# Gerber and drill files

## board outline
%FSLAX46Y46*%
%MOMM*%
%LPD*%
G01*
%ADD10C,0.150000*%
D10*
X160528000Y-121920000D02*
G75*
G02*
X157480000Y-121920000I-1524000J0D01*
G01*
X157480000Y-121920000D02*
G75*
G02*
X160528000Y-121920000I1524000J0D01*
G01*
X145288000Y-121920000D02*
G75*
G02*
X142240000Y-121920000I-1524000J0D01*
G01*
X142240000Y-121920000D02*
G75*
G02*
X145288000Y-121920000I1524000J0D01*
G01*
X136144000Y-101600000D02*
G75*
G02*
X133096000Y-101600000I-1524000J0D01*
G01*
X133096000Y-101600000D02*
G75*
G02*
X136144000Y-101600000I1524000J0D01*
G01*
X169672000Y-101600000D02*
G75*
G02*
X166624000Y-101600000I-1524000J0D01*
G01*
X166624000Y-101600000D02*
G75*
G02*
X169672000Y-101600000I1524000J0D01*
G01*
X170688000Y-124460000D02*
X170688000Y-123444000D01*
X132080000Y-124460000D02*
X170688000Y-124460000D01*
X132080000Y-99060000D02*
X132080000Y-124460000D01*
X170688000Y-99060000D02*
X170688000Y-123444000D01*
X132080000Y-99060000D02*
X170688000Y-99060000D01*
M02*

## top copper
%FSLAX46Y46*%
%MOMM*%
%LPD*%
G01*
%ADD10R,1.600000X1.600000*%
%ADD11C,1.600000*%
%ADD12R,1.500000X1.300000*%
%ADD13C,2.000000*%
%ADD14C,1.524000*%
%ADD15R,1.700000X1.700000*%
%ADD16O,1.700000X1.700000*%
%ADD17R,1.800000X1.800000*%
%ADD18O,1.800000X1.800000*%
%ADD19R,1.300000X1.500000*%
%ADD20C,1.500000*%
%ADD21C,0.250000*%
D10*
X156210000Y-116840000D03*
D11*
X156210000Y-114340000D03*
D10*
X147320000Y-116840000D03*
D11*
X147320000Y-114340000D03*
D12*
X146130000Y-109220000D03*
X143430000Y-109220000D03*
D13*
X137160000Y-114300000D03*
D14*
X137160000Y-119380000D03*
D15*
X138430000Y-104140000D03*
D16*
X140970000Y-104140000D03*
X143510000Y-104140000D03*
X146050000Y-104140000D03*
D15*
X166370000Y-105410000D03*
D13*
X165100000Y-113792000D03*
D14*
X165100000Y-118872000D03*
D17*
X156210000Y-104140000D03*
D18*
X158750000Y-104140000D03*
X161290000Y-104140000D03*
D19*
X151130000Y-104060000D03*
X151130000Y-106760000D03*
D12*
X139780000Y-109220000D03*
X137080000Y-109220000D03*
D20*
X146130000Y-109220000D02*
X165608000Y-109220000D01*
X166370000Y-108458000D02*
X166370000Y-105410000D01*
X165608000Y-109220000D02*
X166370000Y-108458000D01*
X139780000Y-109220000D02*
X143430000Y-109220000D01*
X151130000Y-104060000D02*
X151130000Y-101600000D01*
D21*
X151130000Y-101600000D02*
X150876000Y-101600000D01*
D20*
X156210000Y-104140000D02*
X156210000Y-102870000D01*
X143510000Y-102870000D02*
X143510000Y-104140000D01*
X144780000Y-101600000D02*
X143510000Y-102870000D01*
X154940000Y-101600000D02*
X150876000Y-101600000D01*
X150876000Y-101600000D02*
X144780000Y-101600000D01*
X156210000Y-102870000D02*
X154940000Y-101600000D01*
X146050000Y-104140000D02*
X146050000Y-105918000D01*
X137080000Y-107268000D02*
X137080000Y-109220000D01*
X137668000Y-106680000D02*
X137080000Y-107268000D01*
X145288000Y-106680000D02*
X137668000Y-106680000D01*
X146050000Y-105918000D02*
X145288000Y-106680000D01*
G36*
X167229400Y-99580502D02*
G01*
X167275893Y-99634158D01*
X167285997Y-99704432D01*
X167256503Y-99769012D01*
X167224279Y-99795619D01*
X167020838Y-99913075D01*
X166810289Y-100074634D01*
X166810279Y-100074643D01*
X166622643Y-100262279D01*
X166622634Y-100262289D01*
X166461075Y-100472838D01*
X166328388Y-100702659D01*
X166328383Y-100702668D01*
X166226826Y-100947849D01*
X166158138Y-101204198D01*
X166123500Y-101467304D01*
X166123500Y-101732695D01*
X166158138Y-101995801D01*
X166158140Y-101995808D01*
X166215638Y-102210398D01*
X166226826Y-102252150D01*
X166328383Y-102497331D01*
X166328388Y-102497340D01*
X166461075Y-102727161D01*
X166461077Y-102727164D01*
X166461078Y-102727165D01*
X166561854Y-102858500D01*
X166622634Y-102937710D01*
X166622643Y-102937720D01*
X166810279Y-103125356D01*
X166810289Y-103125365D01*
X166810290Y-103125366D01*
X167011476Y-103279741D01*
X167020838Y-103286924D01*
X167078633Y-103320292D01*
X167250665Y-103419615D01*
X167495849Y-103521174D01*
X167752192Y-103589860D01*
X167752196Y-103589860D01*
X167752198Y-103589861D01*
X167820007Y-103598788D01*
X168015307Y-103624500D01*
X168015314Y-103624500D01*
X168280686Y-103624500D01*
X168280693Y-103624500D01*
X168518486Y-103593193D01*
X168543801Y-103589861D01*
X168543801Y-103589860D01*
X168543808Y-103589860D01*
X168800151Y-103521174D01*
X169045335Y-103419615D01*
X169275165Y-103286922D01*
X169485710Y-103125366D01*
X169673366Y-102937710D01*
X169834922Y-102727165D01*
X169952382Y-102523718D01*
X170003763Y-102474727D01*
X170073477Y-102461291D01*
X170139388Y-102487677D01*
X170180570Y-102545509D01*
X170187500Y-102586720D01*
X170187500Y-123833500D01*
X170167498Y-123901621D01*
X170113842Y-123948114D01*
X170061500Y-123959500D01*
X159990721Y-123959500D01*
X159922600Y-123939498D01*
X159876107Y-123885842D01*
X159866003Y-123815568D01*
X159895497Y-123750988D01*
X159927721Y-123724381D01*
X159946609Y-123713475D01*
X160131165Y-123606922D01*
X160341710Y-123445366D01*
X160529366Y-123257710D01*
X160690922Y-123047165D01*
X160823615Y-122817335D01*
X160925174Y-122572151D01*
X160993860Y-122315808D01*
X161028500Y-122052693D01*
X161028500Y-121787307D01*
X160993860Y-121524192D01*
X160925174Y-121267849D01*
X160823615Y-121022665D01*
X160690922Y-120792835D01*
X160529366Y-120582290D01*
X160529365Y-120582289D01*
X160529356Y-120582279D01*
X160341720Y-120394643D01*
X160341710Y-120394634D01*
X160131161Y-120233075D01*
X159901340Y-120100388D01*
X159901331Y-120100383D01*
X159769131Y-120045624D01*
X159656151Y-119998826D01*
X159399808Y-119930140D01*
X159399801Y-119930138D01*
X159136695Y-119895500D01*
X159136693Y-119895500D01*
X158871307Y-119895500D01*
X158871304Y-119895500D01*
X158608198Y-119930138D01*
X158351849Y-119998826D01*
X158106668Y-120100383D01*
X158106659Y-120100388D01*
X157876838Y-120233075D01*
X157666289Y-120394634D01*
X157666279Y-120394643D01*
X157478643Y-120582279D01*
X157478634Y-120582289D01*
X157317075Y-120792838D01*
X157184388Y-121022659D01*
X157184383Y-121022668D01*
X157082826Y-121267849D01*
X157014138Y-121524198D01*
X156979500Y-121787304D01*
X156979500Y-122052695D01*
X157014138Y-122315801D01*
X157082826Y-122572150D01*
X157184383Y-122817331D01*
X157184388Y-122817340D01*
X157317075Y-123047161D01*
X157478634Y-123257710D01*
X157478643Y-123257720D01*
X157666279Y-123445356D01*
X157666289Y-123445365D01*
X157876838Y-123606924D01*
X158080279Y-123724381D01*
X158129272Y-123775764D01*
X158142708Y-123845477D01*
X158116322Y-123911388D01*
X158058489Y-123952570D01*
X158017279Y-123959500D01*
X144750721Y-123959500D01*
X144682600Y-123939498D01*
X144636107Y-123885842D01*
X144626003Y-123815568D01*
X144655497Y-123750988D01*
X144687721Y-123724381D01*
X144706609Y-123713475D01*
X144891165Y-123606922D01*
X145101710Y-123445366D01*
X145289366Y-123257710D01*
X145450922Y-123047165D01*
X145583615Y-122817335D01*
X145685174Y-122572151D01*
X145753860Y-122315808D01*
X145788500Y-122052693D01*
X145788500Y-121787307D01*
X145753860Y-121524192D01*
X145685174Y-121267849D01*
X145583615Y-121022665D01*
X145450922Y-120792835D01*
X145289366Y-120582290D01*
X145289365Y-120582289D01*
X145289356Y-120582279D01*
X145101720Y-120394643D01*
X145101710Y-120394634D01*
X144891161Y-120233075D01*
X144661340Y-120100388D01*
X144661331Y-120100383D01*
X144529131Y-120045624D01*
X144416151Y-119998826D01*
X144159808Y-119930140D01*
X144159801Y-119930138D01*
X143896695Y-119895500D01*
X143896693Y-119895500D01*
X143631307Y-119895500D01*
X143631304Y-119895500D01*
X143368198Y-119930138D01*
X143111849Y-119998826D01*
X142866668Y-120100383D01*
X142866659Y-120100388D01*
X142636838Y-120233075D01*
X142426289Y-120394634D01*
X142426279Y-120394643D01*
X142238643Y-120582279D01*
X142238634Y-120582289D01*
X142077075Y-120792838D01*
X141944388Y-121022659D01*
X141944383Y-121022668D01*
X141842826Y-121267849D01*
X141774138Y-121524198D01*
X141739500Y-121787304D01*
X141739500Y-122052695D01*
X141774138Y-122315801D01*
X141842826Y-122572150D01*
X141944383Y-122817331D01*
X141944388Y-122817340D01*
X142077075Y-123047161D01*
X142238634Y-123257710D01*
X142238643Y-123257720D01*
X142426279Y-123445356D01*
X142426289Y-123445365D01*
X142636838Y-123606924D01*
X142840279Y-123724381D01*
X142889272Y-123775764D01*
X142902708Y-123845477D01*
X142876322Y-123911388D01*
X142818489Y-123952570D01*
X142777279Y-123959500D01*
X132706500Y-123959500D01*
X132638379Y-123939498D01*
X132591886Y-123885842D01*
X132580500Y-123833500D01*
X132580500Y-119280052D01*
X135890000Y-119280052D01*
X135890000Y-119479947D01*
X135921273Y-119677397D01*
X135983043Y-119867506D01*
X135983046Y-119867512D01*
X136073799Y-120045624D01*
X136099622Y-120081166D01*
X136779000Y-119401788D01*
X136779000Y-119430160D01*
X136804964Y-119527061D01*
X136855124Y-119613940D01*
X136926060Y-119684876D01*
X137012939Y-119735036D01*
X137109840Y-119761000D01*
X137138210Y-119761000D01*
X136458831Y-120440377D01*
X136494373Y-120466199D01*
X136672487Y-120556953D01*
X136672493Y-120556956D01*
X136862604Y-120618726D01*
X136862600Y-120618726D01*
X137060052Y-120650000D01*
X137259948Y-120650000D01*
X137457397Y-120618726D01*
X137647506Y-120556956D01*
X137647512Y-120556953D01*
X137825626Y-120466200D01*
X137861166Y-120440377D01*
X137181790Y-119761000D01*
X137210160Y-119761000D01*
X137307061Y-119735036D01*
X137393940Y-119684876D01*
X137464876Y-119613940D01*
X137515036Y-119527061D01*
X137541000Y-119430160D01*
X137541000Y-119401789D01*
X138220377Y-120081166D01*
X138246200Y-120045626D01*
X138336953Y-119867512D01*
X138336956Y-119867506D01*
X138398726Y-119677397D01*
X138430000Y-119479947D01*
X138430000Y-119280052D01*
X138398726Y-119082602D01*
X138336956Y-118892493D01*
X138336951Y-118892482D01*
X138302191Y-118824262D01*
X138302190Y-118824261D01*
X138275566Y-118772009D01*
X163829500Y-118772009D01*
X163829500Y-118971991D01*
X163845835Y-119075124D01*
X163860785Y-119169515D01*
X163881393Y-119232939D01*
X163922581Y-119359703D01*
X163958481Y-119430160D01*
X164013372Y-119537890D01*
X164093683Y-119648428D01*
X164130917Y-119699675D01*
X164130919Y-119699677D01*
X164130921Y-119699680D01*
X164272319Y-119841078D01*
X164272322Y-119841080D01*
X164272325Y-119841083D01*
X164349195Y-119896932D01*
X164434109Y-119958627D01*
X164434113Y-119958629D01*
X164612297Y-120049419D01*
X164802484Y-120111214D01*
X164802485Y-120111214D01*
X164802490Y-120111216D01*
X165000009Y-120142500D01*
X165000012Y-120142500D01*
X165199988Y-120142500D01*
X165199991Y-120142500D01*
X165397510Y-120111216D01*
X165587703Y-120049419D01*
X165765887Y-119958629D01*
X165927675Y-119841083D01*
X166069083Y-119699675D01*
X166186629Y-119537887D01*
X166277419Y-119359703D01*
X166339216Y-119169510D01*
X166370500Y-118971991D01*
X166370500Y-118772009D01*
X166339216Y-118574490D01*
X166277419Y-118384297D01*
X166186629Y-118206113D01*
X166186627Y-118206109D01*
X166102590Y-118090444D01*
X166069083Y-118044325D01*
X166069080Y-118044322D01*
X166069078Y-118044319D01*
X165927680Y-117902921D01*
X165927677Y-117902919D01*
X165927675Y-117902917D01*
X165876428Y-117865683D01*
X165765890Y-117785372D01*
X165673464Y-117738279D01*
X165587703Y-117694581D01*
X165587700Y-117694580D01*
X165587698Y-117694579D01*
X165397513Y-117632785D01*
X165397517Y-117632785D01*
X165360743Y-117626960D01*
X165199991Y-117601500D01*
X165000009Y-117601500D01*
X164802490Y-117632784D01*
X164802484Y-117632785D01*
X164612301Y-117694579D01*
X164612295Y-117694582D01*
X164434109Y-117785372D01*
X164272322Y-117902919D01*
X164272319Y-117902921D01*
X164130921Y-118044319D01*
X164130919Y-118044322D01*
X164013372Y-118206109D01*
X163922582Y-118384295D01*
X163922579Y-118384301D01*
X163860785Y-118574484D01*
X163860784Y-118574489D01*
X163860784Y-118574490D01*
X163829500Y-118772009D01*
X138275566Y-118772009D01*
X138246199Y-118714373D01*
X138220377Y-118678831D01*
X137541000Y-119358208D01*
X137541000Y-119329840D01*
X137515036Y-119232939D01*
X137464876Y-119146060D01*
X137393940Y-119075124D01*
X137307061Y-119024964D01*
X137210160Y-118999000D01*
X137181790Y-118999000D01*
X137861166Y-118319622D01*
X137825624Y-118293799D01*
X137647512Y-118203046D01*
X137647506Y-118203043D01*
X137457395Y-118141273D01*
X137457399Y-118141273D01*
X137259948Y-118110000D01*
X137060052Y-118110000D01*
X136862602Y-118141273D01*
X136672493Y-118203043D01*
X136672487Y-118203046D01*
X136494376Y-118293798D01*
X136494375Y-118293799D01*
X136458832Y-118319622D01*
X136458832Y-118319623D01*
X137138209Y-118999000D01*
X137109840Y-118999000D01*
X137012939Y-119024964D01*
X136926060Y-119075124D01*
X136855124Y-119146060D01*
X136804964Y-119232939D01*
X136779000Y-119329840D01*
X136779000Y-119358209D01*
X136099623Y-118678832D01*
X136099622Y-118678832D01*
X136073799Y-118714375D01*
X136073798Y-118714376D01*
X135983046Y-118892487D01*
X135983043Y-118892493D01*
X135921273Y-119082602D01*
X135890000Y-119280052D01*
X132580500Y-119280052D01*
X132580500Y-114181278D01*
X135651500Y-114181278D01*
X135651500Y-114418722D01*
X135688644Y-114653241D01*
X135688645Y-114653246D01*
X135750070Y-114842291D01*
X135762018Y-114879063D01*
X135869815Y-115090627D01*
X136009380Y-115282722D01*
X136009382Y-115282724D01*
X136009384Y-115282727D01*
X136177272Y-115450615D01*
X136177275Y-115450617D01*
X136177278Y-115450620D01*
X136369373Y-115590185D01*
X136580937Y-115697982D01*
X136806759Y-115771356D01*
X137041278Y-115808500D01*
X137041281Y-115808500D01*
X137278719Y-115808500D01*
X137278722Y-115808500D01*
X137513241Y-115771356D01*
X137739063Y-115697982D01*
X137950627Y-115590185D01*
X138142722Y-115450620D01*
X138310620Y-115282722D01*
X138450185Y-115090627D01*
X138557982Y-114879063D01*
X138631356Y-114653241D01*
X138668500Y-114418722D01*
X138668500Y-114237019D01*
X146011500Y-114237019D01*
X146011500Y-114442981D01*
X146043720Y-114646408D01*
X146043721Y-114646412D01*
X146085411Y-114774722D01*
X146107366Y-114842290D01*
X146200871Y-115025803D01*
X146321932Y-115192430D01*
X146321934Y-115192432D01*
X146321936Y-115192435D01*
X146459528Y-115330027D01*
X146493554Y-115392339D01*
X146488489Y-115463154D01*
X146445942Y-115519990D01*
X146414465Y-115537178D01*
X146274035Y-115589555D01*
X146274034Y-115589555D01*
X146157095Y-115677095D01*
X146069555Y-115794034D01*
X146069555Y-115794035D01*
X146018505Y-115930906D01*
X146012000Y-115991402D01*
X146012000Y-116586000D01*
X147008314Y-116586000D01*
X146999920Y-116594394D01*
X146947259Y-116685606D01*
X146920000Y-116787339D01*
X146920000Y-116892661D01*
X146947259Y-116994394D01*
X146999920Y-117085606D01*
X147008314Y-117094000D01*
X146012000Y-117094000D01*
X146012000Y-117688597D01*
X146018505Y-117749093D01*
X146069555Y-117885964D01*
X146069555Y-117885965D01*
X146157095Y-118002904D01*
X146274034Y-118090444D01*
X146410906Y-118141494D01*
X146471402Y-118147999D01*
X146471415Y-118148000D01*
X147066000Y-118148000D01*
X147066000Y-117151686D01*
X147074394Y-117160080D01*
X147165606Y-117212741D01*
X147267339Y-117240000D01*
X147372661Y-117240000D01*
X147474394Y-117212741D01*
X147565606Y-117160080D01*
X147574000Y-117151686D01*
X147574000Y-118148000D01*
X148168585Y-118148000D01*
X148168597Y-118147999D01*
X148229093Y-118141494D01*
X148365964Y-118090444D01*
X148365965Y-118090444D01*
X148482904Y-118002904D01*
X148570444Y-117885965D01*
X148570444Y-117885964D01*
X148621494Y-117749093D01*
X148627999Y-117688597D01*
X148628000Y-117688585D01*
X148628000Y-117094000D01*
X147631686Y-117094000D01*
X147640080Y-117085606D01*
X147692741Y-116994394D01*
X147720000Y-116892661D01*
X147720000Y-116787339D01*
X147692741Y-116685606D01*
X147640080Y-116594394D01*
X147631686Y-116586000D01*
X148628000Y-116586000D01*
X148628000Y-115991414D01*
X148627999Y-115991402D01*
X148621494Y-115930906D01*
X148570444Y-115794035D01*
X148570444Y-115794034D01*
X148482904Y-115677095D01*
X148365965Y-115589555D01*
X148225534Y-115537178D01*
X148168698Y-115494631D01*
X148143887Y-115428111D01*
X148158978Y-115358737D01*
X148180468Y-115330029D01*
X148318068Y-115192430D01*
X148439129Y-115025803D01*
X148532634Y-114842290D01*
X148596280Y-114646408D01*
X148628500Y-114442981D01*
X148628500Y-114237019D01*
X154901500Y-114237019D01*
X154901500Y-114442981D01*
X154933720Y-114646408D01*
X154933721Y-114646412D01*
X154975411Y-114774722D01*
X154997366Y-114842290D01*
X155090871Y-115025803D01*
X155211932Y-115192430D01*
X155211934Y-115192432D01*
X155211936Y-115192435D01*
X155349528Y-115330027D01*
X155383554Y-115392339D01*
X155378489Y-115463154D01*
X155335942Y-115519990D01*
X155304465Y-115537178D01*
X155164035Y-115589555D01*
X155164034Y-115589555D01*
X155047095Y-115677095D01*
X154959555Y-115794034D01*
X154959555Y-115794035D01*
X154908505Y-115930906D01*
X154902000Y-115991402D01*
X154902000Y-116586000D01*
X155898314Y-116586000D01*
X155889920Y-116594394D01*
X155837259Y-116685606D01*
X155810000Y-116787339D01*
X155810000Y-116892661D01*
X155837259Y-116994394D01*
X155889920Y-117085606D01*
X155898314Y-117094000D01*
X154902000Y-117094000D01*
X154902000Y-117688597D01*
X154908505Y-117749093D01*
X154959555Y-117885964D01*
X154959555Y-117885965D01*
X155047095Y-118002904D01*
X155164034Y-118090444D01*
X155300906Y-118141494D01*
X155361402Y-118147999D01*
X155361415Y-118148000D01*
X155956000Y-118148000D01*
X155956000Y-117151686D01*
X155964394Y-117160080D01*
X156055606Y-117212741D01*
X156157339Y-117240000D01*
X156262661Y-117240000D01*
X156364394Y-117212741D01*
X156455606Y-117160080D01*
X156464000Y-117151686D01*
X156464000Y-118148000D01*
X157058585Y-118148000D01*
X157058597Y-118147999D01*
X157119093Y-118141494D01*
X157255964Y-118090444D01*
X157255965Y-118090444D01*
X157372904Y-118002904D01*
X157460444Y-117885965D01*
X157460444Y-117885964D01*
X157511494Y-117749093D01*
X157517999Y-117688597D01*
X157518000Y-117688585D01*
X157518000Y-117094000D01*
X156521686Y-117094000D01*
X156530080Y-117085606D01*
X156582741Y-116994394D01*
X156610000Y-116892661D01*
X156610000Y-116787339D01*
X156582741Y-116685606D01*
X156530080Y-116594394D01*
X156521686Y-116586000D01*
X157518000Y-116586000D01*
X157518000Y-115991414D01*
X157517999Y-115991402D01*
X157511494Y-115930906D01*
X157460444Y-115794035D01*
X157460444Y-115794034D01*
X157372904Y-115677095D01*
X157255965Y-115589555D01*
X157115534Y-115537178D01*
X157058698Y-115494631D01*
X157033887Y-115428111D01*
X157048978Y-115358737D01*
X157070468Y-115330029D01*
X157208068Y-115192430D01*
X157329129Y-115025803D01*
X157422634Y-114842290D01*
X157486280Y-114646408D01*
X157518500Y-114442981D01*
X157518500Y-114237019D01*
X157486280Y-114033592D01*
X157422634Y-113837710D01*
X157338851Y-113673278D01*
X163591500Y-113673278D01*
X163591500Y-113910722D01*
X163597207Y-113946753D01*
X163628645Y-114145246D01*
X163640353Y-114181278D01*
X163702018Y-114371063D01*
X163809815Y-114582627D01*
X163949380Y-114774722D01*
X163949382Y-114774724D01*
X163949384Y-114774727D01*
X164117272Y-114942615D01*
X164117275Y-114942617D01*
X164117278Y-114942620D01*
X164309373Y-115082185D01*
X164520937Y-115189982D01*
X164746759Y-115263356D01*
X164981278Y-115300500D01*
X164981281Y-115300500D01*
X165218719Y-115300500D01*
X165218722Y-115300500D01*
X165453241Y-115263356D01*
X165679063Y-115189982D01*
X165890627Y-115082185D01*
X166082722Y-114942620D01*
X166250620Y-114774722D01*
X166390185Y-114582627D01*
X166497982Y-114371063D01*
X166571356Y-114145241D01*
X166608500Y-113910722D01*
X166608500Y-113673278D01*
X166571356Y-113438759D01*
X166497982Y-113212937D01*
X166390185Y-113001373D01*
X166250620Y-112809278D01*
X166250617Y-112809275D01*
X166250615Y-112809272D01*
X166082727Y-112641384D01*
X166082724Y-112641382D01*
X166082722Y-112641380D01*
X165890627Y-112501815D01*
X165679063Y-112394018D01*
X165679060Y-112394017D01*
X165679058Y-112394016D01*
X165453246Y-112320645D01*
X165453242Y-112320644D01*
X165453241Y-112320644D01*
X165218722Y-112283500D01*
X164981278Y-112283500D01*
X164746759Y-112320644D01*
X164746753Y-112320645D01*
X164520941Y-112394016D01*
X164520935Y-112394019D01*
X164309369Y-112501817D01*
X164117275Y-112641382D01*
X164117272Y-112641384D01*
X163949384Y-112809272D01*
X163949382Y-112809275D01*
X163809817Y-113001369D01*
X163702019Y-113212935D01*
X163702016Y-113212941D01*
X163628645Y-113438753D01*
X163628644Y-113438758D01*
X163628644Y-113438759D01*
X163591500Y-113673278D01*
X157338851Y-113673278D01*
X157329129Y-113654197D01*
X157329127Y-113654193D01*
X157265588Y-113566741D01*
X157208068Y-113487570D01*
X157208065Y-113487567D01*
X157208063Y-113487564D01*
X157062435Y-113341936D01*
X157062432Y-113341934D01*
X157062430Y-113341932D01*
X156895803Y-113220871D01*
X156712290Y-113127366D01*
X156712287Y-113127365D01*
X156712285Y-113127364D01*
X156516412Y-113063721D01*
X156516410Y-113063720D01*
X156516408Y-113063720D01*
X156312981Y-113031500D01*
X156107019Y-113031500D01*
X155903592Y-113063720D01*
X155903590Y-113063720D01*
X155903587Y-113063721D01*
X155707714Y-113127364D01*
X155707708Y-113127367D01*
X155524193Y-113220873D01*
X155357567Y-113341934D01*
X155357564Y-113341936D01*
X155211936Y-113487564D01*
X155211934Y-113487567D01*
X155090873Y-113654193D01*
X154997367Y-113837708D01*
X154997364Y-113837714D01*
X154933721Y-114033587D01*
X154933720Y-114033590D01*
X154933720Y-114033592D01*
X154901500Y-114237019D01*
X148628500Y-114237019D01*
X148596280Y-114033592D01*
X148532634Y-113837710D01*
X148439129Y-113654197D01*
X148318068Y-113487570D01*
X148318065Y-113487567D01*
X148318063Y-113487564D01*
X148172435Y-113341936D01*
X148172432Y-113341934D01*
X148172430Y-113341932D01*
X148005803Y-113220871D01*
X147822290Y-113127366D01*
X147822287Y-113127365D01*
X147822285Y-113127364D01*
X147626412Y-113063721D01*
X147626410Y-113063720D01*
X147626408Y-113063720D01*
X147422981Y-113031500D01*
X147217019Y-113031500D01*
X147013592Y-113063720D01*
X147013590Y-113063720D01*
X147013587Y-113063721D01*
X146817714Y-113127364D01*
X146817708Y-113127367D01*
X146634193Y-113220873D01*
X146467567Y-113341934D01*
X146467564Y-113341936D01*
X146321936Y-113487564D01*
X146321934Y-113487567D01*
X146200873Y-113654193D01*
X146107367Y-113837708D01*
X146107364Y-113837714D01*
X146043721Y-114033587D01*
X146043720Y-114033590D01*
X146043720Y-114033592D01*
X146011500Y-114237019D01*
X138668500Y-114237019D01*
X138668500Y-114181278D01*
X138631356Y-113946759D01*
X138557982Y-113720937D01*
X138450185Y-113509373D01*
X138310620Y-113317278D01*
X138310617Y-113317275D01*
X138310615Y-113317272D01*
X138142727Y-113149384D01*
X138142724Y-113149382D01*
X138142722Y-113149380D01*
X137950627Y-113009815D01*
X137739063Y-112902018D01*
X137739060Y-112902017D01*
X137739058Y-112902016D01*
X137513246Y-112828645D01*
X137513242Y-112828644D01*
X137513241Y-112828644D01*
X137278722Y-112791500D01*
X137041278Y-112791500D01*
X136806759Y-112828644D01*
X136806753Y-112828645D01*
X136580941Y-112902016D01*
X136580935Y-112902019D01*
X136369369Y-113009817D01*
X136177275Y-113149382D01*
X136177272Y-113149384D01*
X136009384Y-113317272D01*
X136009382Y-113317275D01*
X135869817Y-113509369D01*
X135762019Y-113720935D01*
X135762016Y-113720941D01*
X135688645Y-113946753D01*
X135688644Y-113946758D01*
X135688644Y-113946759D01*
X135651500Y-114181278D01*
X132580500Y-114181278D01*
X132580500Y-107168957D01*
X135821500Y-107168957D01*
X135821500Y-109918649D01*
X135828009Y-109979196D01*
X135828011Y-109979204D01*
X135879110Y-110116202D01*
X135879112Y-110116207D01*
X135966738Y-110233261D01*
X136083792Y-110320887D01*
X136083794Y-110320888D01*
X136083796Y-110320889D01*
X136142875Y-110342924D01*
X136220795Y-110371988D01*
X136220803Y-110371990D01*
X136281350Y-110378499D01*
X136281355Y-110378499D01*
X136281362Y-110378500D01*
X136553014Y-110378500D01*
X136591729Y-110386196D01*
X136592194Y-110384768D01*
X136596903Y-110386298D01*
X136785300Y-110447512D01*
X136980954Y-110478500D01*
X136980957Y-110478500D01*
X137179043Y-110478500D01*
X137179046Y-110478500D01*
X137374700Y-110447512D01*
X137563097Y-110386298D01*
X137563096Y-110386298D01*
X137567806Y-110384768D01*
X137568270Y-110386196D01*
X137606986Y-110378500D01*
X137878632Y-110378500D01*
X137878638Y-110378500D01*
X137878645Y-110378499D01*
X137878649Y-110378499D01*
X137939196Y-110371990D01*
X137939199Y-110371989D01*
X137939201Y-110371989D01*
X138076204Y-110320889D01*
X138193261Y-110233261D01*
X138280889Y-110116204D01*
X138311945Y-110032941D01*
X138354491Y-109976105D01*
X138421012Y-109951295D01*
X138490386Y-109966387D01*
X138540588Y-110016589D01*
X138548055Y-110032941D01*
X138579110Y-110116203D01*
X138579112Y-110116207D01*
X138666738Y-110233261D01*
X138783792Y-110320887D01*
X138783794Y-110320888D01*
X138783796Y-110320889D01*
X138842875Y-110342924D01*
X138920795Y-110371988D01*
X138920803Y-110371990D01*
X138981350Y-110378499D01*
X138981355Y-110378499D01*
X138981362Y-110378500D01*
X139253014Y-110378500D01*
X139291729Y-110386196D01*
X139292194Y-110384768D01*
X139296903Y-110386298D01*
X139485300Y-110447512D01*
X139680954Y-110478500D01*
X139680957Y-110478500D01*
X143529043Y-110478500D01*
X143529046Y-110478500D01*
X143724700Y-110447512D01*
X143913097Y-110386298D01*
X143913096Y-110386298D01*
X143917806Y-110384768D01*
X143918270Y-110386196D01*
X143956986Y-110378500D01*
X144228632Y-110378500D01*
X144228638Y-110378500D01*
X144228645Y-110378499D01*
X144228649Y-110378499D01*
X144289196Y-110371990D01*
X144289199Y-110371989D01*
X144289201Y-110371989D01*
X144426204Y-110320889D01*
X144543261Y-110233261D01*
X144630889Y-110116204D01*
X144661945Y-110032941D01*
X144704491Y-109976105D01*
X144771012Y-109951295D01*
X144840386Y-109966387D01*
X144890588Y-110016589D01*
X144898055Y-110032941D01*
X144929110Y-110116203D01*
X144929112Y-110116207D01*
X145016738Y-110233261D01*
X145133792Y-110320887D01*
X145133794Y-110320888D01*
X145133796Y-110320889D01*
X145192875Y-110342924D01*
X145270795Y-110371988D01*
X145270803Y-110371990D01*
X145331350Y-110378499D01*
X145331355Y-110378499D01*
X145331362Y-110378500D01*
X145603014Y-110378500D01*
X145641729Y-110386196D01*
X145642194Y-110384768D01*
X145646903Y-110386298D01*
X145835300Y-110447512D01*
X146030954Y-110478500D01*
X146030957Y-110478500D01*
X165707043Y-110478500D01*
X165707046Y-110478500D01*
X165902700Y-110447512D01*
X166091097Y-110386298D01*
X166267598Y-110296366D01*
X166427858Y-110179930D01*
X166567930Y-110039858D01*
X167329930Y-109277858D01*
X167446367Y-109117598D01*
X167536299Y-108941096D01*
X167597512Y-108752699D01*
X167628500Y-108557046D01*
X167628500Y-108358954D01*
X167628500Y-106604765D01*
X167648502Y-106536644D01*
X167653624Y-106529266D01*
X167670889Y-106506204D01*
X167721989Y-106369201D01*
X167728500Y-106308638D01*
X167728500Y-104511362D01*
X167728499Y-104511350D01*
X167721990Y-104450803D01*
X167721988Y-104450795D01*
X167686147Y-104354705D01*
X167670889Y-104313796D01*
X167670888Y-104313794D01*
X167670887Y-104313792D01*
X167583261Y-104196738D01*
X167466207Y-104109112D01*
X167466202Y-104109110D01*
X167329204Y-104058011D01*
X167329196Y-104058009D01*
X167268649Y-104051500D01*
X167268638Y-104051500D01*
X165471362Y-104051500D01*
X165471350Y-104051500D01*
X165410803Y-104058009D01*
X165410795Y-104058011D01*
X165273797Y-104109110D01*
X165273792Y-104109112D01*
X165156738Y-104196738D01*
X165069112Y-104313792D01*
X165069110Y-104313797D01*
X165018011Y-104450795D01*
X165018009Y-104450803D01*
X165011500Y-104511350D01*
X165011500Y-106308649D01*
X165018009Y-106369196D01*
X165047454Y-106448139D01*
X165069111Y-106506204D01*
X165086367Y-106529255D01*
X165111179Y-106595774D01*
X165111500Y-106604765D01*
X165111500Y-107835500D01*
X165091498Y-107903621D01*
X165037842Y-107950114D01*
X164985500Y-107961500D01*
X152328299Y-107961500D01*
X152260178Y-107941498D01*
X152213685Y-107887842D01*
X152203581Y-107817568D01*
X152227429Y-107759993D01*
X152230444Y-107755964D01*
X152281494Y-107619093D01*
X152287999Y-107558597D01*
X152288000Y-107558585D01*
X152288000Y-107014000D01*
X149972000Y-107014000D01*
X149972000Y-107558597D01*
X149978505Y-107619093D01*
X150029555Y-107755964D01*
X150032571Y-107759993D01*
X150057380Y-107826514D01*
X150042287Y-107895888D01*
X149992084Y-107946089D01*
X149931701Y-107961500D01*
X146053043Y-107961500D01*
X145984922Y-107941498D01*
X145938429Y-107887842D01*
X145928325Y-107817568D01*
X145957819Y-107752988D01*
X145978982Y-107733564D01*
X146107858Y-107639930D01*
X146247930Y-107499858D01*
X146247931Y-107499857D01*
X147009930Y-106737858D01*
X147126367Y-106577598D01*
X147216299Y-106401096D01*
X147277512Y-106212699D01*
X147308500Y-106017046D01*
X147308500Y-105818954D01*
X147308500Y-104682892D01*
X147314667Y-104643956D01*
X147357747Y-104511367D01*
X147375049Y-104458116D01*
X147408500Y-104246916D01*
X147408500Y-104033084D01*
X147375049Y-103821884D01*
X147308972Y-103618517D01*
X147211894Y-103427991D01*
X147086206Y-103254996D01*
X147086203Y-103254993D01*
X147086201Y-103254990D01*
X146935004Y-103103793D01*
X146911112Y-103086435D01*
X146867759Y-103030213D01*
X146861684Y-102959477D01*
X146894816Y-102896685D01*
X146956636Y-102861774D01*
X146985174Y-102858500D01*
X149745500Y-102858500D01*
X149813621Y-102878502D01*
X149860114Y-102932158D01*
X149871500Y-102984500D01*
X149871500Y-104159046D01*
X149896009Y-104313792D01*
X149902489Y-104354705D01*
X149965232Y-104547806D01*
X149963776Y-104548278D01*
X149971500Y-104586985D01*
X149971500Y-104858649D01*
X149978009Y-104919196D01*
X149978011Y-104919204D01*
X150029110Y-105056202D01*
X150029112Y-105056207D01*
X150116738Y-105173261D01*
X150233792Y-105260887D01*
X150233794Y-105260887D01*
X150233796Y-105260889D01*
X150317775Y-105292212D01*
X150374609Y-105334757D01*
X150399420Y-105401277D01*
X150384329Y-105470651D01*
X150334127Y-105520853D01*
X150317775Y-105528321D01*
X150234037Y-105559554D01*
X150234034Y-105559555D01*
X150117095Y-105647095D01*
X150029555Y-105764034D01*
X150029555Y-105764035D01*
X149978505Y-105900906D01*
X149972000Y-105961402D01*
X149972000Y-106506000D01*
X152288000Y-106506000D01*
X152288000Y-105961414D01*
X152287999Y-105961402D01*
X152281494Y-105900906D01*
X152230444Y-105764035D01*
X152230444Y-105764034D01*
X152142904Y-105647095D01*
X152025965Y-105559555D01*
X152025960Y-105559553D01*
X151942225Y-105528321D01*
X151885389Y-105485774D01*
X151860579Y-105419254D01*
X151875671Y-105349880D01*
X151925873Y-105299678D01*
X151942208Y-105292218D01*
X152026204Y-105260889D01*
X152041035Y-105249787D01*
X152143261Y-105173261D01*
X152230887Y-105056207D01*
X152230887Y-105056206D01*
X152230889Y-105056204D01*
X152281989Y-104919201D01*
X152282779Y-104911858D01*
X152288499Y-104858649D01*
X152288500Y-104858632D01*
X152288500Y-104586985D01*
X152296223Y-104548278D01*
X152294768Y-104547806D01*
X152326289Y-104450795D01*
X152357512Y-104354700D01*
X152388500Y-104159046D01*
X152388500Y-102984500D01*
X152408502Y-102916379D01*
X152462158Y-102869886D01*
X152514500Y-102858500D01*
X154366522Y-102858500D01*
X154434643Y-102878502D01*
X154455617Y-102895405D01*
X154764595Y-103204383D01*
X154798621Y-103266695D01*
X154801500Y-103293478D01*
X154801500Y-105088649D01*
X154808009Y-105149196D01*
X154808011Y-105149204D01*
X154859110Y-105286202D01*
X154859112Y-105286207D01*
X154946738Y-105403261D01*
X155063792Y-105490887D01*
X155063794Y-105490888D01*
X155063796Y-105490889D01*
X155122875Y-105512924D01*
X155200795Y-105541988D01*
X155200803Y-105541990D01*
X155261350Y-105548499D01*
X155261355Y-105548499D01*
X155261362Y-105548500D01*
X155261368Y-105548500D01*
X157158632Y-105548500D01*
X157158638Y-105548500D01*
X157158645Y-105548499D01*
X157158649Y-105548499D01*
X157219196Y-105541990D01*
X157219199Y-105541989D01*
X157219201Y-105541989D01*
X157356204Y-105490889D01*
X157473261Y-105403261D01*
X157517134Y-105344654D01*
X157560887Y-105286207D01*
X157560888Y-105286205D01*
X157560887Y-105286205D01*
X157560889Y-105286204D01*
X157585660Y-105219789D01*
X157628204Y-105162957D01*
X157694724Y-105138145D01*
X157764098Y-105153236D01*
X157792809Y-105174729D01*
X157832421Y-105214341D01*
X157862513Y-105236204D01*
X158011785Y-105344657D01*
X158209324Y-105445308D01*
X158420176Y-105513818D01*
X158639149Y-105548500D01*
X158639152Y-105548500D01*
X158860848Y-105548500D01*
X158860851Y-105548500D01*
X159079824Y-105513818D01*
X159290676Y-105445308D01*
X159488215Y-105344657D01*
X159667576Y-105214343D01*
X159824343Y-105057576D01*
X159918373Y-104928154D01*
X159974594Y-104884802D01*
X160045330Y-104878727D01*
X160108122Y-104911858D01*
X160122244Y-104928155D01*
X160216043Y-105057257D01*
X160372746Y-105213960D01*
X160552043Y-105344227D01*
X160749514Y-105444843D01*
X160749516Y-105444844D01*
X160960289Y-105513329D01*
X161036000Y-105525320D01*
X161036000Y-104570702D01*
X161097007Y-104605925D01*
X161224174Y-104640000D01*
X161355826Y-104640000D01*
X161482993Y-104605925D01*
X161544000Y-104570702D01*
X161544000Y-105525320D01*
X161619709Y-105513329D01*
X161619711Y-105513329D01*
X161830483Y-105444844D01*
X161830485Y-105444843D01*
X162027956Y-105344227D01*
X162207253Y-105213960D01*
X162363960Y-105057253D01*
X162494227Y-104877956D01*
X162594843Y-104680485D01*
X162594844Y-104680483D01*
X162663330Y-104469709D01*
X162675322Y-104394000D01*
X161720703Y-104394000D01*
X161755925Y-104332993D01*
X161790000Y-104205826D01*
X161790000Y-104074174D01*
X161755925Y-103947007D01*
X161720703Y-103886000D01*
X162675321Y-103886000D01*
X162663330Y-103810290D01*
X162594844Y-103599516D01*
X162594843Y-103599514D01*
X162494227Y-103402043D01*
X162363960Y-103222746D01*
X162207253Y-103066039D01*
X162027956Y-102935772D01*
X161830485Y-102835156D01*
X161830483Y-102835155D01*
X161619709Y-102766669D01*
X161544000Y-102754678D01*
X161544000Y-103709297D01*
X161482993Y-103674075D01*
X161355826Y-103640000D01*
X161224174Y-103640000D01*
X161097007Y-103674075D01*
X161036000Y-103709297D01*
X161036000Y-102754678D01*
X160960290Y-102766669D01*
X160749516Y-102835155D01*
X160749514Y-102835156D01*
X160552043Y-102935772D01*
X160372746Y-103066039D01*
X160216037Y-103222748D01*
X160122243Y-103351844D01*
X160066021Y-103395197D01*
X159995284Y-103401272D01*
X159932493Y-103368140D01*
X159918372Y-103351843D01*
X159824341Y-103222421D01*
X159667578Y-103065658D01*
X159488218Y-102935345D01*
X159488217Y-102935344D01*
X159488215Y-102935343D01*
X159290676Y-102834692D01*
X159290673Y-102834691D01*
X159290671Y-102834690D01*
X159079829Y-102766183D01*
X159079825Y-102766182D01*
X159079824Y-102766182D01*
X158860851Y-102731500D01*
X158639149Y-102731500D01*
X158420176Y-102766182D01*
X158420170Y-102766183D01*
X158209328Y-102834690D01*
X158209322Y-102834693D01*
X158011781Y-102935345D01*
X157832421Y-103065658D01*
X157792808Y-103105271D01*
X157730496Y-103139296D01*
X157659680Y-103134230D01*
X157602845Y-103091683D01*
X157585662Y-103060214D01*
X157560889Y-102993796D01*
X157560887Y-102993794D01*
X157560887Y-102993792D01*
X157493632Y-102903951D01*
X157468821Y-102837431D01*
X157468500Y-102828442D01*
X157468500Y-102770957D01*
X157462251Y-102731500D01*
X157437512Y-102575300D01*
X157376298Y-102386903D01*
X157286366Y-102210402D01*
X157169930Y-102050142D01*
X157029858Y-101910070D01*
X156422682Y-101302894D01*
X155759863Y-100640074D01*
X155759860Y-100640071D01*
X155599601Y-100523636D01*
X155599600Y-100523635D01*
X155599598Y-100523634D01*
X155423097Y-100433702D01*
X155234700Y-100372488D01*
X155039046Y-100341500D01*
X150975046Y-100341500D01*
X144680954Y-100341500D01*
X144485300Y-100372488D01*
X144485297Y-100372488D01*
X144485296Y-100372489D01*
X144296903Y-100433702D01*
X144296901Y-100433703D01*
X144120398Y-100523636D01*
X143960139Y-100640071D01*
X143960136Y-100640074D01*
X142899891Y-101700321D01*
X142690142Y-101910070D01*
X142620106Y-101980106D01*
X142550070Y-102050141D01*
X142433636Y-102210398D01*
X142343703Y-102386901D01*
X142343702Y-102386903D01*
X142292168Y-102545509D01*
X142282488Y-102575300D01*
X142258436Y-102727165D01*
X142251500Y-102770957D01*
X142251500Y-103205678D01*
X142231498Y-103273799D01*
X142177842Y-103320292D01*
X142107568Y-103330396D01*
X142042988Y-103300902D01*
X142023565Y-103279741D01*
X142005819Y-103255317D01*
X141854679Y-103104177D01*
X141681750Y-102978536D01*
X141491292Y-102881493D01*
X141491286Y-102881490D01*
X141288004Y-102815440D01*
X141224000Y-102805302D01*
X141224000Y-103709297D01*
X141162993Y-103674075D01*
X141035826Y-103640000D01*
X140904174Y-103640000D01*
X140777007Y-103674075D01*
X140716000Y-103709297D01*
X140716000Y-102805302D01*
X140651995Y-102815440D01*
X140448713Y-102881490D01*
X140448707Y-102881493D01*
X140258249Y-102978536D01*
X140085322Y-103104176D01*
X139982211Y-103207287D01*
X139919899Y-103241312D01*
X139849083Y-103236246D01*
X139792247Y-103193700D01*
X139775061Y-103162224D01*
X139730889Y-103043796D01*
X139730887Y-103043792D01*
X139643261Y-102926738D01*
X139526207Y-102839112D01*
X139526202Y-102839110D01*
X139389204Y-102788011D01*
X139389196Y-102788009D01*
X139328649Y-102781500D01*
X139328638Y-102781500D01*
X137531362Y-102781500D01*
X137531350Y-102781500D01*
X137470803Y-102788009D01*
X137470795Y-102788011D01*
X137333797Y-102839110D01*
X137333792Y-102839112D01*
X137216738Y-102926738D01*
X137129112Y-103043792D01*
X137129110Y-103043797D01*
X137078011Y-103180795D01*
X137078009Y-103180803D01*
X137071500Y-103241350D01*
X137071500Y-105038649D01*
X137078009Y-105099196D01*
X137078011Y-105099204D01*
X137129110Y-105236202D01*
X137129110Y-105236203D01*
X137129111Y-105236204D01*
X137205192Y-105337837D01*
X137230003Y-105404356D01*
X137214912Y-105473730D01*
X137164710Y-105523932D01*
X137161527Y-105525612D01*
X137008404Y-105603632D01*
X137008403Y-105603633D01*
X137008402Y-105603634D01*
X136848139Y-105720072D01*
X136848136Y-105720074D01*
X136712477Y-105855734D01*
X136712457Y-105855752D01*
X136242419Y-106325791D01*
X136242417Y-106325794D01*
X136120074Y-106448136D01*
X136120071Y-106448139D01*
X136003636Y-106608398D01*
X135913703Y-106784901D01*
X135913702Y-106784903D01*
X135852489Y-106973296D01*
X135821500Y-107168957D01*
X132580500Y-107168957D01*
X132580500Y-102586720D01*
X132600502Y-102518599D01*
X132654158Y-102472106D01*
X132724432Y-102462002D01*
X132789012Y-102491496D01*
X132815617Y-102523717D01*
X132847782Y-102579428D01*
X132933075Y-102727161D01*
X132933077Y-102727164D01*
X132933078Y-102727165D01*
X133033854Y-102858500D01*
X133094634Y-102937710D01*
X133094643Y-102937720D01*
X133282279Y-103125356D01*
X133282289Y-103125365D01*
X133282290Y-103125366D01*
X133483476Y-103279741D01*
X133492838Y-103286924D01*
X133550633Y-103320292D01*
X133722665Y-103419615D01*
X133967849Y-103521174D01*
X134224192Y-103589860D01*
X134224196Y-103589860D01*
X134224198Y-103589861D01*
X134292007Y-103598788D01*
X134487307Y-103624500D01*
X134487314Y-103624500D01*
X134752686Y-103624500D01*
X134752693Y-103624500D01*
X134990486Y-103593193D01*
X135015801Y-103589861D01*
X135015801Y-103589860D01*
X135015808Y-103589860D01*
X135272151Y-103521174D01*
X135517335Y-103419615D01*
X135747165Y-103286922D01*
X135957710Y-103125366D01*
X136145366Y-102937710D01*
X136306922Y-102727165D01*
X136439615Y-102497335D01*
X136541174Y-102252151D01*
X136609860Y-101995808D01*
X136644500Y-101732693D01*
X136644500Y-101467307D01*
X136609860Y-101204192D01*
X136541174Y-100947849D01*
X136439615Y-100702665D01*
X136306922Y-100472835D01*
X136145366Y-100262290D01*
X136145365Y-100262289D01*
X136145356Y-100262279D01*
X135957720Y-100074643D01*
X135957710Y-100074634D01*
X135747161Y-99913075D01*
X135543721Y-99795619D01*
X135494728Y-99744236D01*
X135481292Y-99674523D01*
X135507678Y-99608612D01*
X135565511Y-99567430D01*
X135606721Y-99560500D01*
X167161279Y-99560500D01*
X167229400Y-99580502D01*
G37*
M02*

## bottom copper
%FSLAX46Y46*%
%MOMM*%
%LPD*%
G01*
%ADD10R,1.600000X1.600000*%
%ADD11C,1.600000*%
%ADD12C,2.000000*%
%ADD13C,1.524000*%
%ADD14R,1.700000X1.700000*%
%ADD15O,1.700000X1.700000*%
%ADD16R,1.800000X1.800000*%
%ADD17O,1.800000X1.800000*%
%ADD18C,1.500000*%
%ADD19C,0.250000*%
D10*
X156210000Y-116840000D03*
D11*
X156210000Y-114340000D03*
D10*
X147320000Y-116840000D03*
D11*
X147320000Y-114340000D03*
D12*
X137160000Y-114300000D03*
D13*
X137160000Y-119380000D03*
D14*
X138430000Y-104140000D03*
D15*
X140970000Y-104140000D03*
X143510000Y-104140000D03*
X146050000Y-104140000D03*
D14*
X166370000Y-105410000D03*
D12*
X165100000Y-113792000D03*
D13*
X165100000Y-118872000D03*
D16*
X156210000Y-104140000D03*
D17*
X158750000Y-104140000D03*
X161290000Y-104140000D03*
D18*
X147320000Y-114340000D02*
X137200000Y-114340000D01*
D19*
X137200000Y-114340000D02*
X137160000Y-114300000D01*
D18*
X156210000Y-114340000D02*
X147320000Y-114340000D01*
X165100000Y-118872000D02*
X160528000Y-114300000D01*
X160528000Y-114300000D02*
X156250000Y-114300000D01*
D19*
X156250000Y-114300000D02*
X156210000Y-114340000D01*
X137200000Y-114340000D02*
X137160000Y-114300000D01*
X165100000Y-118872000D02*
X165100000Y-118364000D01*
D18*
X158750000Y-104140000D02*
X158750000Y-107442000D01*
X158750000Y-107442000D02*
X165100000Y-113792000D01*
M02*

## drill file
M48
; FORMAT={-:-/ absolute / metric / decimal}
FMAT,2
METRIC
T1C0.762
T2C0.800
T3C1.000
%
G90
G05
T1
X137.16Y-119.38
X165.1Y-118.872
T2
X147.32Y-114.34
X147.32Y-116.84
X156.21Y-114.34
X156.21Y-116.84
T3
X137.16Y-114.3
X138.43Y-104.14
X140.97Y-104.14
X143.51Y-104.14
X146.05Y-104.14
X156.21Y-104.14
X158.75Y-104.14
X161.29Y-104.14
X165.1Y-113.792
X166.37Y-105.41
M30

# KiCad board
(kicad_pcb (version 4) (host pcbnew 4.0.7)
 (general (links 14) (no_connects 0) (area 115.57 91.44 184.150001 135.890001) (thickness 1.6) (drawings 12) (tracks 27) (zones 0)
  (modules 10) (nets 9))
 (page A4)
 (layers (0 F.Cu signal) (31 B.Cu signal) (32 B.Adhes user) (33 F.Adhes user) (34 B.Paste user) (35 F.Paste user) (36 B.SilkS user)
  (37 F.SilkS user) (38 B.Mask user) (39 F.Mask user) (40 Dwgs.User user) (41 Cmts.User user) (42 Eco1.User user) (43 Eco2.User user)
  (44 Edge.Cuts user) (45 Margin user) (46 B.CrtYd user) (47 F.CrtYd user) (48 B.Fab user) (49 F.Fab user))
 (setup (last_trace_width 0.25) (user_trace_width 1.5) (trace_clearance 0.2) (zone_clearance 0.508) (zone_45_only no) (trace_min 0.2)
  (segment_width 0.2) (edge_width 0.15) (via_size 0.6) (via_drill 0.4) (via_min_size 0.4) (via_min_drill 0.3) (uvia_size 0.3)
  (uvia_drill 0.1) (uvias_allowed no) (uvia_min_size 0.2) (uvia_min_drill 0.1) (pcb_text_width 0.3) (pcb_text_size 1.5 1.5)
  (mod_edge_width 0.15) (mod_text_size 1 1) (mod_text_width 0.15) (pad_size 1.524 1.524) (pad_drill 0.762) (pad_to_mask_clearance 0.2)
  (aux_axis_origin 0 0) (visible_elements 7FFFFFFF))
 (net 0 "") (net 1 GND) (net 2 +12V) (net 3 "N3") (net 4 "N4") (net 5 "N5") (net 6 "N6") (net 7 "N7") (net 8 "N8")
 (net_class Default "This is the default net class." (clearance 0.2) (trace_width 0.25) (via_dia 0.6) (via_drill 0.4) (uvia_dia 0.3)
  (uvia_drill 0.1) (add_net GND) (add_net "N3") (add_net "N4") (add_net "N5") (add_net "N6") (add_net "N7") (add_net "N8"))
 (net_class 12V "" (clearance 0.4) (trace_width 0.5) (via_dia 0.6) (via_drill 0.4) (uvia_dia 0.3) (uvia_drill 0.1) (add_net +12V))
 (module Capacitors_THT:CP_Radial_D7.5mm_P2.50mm (layer F.Cu) (at 156.21 116.84 90)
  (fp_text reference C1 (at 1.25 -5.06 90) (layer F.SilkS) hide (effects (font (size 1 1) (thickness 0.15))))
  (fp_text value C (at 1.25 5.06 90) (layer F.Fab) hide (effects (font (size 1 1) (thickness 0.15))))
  (pad 1 thru_hole rect (at 0 0 90) (size 1.6 1.6) (drill 0.8) (layers *.Cu *.Mask) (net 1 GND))
  (pad 2 thru_hole circle (at 2.5 0 90) (size 1.6 1.6) (drill 0.8) (layers *.Cu *.Mask) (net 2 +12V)))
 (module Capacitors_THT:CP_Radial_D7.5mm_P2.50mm (layer F.Cu) (at 147.32 116.84 90)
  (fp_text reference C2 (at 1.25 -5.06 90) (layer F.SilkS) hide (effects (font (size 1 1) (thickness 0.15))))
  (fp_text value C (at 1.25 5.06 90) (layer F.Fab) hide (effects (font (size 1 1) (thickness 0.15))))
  (pad 1 thru_hole rect (at 0 0 90) (size 1.6 1.6) (drill 0.8) (layers *.Cu *.Mask) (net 1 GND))
  (pad 2 thru_hole circle (at 2.5 0 90) (size 1.6 1.6) (drill 0.8) (layers *.Cu *.Mask) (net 2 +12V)))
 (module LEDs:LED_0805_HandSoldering (layer F.Cu) (at 144.78 109.22 180)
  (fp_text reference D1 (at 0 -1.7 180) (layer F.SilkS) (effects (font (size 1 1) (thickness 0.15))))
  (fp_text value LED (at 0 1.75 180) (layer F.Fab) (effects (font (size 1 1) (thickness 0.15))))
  (pad 1 smd rect (at -1.35 0 180) (size 1.5 1.3) (layers F.Cu F.Paste F.Mask) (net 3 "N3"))
  (pad 2 smd rect (at 1.35 0 180) (size 1.5 1.3) (layers F.Cu F.Paste F.Mask) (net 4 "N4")))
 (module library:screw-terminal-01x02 (layer F.Cu) (at 137.16 116.84)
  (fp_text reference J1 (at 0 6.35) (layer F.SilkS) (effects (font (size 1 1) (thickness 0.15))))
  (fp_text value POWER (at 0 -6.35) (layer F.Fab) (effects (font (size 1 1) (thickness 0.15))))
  (pad 1 thru_hole circle (at 0 -2.54) (size 2 2) (drill 1) (layers *.Cu *.Mask) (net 2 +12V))
  (pad 2 thru_hole circle (at 0 2.54) (size 1.524 1.524) (drill 0.762) (layers *.Cu *.Mask) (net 1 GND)))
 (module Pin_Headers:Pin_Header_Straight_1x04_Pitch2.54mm (layer F.Cu) (at 138.43 104.14 90)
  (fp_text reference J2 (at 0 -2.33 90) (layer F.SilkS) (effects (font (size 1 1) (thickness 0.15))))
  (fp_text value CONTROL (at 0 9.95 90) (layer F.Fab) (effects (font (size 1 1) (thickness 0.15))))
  (pad 1 thru_hole rect (at 0 0 90) (size 1.7 1.7) (drill 1) (layers *.Cu *.Mask) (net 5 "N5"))
  (pad 2 thru_hole oval (at 0 2.54 90) (size 1.7 1.7) (drill 1) (layers *.Cu *.Mask) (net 1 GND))
  (pad 3 thru_hole oval (at 0 5.08 90) (size 1.7 1.7) (drill 1) (layers *.Cu *.Mask) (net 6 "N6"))
  (pad 4 thru_hole oval (at 0 7.62 90) (size 1.7 1.7) (drill 1) (layers *.Cu *.Mask) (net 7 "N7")))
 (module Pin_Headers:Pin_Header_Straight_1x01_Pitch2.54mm (layer F.Cu) (at 166.37 105.41)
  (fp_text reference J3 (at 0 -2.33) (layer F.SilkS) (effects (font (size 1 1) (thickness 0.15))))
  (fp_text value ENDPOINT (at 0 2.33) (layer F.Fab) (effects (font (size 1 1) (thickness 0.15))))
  (pad 1 thru_hole rect (at 0 0) (size 1.7 1.7) (drill 1) (layers *.Cu *.Mask) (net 3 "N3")))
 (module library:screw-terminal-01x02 (layer F.Cu) (at 165.1 116.332)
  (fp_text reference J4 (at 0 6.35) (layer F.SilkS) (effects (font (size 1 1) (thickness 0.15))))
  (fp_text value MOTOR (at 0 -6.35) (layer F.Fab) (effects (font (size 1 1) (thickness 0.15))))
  (pad 1 thru_hole circle (at 0 -2.54) (size 2 2) (drill 1) (layers *.Cu *.Mask) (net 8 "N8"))
  (pad 2 thru_hole circle (at 0 2.54) (size 1.524 1.524) (drill 0.762) (layers *.Cu *.Mask) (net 2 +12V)))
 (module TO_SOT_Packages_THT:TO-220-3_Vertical (layer F.Cu) (at 156.21 104.14)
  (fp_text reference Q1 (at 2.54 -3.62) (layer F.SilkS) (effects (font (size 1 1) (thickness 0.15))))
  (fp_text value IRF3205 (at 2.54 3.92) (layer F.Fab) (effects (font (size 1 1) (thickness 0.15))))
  (pad 1 thru_hole rect (at 0 0) (size 1.8 1.8) (drill 1) (layers *.Cu *.Mask) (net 6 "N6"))
  (pad 2 thru_hole oval (at 2.54 0) (size 1.8 1.8) (drill 1) (layers *.Cu *.Mask) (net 8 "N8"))
  (pad 3 thru_hole oval (at 5.08 0) (size 1.8 1.8) (drill 1) (layers *.Cu *.Mask) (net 1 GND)))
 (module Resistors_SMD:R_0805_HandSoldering (layer F.Cu) (at 151.13 105.41 270)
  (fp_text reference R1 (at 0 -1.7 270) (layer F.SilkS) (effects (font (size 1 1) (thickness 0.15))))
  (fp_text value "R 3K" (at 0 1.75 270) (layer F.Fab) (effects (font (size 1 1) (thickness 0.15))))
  (pad 1 smd rect (at -1.35 0 270) (size 1.5 1.3) (layers F.Cu F.Paste F.Mask) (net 6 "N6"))
  (pad 2 smd rect (at 1.35 0 270) (size 1.5 1.3) (layers F.Cu F.Paste F.Mask) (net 1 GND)))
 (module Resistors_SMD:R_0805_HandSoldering (layer F.Cu) (at 138.43 109.22 180)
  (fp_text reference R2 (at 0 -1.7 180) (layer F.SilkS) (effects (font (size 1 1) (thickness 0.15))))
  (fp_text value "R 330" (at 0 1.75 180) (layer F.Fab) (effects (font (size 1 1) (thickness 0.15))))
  (pad 1 smd rect (at -1.35 0 180) (size 1.5 1.3) (layers F.Cu F.Paste F.Mask) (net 4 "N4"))
  (pad 2 smd rect (at 1.35 0 180) (size 1.5 1.3) (layers F.Cu F.Paste F.Mask) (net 7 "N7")))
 (gr_circle (center 159.004 121.92) (end 159.004 120.396) (layer Edge.Cuts) (width 0.15))
 (gr_circle (center 143.764 121.92) (end 143.764 120.396) (layer Edge.Cuts) (width 0.15))
 (gr_circle (center 134.62 101.6) (end 134.62 100.076) (layer Edge.Cuts) (width 0.15))
 (gr_circle (center 168.148 101.6) (end 168.148 100.076) (layer Edge.Cuts) (width 0.15))
 (gr_line (start 170.688 124.46) (end 170.688 123.444) (angle 90) (layer Edge.Cuts) (width 0.15))
 (gr_line (start 132.08 124.46) (end 170.688 124.46) (angle 90) (layer Edge.Cuts) (width 0.15))
 (gr_line (start 132.08 99.06) (end 132.08 124.46) (angle 90) (layer Edge.Cuts) (width 0.15))
 (gr_line (start 170.688 99.06) (end 170.688 123.444) (angle 90) (layer Edge.Cuts) (width 0.15))
 (gr_line (start 132.08 99.06) (end 170.688 99.06) (angle 90) (layer Edge.Cuts) (width 0.15))
 (segment (start 147.32 114.34) (end 137.2 114.34) (width 1.5) (layer B.Cu) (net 2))
 (segment (start 137.2 114.34) (end 137.16 114.3) (width 0.25) (layer B.Cu) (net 2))
 (segment (start 156.21 114.34) (end 147.32 114.34) (width 1.5) (layer B.Cu) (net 2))
 (segment (start 165.1 118.872) (end 160.528 114.3) (width 1.5) (layer B.Cu) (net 2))
 (segment (start 160.528 114.3) (end 156.25 114.3) (width 1.5) (layer B.Cu) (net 2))
 (segment (start 156.25 114.3) (end 156.21 114.34) (width 0.25) (layer B.Cu) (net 2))
 (segment (start 137.2 114.34) (end 137.16 114.3) (width 0.25) (layer B.Cu) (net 2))
 (segment (start 165.1 118.872) (end 165.1 118.364) (width 0.25) (layer B.Cu) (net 2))
 (segment (start 146.13 109.22) (end 165.608 109.22) (width 1.5) (layer F.Cu) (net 3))
 (segment (start 166.37 108.458) (end 166.37 105.41) (width 1.5) (layer F.Cu) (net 3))
 (segment (start 165.608 109.22) (end 166.37 108.458) (width 1.5) (layer F.Cu) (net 3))
 (segment (start 139.78 109.22) (end 143.43 109.22) (width 1.5) (layer F.Cu) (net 4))
 (segment (start 151.13 104.06) (end 151.13 101.6) (width 1.5) (layer F.Cu) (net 6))
 (segment (start 151.13 101.6) (end 150.876 101.6) (width 0.25) (layer F.Cu) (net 6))
 (segment (start 156.21 104.14) (end 156.21 102.87) (width 1.5) (layer F.Cu) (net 6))
 (segment (start 143.51 102.87) (end 143.51 104.14) (width 1.5) (layer F.Cu) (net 6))
 (segment (start 144.78 101.6) (end 143.51 102.87) (width 1.5) (layer F.Cu) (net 6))
 (segment (start 154.94 101.6) (end 150.876 101.6) (width 1.5) (layer F.Cu) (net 6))
 (segment (start 150.876 101.6) (end 144.78 101.6) (width 1.5) (layer F.Cu) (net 6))
 (segment (start 156.21 102.87) (end 154.94 101.6) (width 1.5) (layer F.Cu) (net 6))
 (segment (start 146.05 104.14) (end 146.05 105.918) (width 1.5) (layer F.Cu) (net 7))
 (segment (start 137.08 107.268) (end 137.08 109.22) (width 1.5) (layer F.Cu) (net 7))
 (segment (start 137.668 106.68) (end 137.08 107.268) (width 1.5) (layer F.Cu) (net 7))
 (segment (start 145.288 106.68) (end 137.668 106.68) (width 1.5) (layer F.Cu) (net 7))
 (segment (start 146.05 105.918) (end 145.288 106.68) (width 1.5) (layer F.Cu) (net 7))
 (segment (start 158.75 104.14) (end 158.75 107.442) (width 1.5) (layer B.Cu) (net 8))
 (segment (start 158.75 107.442) (end 165.1 113.792) (width 1.5) (layer B.Cu) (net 8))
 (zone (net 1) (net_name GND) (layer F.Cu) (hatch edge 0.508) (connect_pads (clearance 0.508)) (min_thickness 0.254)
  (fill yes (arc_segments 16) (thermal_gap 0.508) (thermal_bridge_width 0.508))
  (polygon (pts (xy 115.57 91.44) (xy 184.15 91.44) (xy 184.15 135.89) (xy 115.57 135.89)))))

